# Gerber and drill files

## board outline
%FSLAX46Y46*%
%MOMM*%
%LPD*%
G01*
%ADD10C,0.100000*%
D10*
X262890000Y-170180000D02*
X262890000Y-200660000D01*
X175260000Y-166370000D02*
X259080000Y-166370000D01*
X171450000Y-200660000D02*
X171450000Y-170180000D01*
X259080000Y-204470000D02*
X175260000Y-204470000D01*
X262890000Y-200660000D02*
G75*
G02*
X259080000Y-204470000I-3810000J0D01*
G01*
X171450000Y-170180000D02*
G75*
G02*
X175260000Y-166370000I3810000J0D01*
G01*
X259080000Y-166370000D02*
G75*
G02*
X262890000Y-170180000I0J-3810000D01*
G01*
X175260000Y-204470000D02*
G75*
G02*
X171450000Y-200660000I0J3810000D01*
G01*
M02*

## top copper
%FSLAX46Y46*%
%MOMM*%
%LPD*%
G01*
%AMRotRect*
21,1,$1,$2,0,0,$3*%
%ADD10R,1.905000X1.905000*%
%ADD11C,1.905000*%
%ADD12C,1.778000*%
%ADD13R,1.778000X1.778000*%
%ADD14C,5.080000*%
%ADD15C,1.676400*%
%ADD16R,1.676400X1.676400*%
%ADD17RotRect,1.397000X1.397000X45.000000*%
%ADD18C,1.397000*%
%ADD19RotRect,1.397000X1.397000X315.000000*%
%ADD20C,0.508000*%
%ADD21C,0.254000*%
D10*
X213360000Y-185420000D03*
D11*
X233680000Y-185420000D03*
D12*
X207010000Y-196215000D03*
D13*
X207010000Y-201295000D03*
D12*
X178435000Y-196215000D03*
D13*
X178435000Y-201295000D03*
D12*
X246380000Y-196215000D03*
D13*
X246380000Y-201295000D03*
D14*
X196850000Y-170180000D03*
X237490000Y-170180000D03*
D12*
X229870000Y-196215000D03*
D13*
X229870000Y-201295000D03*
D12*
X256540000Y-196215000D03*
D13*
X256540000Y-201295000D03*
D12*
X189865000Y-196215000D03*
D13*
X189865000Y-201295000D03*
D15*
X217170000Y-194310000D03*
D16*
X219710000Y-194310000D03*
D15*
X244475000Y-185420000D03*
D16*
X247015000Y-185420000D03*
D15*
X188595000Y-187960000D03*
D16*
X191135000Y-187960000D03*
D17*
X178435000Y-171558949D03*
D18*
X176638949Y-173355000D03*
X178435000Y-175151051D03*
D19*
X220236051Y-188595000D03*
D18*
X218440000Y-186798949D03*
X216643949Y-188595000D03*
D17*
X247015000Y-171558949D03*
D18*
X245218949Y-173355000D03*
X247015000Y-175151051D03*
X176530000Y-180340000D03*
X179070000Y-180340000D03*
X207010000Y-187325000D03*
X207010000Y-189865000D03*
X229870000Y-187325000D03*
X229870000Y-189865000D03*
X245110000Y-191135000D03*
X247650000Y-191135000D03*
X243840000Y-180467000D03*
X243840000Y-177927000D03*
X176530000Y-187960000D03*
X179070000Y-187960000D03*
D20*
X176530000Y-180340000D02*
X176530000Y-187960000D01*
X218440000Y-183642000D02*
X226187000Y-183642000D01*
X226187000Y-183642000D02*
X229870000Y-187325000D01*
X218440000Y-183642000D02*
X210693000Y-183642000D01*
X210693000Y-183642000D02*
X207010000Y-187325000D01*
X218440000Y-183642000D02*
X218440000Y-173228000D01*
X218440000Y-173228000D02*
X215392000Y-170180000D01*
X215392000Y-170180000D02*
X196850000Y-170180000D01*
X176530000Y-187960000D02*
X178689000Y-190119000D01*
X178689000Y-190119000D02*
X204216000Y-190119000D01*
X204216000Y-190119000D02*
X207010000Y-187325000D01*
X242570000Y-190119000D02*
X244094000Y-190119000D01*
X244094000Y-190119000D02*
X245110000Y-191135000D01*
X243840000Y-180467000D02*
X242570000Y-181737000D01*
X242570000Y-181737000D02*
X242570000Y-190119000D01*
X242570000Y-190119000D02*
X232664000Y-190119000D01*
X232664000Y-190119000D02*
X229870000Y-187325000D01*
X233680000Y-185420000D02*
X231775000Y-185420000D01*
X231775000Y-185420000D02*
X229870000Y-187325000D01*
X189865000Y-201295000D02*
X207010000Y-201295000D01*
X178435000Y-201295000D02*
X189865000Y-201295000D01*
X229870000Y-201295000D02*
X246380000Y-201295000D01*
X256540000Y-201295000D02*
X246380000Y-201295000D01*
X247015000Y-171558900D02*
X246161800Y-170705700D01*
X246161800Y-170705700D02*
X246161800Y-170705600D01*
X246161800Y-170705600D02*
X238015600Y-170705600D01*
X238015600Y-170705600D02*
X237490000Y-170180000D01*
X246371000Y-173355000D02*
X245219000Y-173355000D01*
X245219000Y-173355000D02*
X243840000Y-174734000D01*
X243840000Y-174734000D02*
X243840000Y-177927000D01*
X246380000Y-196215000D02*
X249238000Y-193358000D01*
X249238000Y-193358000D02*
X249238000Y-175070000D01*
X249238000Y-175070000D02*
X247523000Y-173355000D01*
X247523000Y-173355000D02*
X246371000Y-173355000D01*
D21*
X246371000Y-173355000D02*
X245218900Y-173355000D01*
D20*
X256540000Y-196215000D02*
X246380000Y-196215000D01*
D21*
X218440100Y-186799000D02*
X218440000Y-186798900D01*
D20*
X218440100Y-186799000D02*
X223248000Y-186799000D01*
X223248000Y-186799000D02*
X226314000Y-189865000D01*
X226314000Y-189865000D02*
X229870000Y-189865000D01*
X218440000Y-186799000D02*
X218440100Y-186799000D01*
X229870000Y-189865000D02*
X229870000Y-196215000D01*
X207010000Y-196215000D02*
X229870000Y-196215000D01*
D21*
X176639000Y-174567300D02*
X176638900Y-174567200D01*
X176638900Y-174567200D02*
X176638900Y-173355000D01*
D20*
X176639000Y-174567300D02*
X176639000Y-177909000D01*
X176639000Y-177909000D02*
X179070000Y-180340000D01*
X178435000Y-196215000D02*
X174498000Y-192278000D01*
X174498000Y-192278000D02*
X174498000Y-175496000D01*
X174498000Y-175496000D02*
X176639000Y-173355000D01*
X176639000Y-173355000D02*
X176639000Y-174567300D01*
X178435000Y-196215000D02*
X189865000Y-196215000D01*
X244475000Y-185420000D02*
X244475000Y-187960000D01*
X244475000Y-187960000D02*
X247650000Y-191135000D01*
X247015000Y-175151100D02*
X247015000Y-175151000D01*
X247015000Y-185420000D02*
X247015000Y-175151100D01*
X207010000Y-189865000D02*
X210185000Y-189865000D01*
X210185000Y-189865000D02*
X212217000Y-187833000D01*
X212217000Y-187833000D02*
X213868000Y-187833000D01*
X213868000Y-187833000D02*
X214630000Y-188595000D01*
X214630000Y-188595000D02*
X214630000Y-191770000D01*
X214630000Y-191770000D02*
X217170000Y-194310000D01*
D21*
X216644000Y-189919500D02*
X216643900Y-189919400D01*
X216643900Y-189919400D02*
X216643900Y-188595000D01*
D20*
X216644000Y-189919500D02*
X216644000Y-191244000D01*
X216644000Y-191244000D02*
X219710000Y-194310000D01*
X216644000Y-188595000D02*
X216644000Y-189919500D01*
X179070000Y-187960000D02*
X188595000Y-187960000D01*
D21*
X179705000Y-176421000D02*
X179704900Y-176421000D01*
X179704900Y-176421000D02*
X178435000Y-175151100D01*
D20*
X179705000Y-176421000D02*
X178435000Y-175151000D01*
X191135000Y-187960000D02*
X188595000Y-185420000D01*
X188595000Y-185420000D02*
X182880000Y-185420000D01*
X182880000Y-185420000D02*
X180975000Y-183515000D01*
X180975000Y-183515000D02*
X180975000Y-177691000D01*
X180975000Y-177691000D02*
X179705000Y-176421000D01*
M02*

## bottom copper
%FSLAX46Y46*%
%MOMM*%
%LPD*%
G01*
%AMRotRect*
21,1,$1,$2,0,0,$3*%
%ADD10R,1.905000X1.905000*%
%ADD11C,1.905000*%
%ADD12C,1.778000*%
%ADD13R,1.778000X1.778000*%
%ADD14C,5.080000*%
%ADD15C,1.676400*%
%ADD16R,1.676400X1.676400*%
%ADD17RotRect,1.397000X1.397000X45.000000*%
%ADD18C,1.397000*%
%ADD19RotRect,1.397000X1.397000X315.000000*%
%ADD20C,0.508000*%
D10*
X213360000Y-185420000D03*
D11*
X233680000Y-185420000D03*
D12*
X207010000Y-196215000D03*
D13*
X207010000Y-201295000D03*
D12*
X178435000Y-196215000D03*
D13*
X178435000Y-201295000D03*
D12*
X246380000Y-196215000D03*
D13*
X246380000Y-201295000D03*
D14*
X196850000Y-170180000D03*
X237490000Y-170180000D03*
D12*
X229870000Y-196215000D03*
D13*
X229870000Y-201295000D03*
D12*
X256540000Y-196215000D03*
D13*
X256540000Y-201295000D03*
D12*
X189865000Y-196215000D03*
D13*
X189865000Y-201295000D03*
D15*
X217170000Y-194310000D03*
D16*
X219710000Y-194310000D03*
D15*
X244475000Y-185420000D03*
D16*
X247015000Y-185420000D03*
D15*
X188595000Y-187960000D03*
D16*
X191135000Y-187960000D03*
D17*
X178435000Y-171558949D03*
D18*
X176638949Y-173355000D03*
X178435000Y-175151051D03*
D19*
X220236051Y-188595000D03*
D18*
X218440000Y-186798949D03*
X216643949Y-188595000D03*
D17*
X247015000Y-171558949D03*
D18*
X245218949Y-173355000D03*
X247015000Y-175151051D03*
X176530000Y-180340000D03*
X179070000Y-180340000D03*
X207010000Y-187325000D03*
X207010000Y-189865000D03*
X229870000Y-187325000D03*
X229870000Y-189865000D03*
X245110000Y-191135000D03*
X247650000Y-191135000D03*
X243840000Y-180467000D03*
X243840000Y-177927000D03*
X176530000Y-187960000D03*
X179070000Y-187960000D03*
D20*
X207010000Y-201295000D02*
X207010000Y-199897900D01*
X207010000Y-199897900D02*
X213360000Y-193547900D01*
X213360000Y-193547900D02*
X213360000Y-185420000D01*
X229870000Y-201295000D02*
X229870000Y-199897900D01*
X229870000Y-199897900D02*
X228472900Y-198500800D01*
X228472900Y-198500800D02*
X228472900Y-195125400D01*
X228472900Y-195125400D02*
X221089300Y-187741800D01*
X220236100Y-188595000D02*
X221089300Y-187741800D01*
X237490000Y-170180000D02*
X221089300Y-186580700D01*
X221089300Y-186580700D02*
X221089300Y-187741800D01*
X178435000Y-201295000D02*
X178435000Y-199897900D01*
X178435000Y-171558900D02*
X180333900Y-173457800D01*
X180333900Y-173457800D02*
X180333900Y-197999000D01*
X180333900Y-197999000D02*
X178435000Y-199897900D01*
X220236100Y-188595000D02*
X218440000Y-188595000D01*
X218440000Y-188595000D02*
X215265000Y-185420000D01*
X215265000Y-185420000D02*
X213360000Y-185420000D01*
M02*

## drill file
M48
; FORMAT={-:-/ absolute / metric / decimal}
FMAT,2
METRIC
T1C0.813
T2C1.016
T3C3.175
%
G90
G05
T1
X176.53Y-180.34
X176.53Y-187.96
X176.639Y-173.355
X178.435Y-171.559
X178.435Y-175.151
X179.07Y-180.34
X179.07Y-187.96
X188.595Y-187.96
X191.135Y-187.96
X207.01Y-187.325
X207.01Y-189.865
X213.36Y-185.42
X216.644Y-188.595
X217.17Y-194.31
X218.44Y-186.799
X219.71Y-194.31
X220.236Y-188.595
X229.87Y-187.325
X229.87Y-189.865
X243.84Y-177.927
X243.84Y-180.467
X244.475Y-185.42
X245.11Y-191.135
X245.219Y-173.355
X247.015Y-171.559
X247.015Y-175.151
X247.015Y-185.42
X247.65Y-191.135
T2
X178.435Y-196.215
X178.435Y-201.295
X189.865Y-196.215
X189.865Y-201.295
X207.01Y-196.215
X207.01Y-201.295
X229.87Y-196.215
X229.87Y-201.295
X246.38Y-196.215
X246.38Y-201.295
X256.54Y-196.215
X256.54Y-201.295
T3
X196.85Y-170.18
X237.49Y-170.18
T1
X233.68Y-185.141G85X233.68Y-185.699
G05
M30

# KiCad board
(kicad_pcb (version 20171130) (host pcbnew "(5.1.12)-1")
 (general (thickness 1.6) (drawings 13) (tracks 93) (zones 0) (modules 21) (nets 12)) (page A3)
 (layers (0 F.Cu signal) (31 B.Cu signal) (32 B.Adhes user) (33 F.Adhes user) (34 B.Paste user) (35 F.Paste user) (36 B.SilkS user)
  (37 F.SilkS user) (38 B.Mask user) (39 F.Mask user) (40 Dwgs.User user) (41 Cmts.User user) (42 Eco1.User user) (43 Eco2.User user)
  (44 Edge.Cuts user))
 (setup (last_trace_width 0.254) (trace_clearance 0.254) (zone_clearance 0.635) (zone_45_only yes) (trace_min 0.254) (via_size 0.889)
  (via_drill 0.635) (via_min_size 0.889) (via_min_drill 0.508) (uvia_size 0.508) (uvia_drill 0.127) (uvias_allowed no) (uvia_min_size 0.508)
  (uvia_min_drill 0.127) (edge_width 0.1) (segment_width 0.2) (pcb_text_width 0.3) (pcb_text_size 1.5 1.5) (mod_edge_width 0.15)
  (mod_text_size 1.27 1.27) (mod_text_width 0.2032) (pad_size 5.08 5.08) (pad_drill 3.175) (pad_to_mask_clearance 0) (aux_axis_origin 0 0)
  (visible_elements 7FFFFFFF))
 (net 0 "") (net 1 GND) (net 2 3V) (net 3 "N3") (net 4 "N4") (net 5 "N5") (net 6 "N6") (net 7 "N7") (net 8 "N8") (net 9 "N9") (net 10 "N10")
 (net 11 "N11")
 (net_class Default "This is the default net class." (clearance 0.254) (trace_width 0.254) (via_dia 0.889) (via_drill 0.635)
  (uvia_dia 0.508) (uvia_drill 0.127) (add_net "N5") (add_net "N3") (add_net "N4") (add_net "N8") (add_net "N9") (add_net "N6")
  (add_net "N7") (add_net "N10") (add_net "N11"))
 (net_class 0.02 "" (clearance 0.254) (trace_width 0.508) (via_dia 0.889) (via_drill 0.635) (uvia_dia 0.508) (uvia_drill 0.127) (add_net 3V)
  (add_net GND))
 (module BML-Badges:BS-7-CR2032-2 (layer B.Cu) (at 217.17 185.42)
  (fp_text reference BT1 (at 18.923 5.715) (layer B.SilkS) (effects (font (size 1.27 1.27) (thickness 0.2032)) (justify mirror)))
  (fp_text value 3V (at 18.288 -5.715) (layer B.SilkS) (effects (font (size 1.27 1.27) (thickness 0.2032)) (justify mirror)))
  (pad 2 thru_hole rect (at -3.81 0) (size 1.905 1.905) (drill 0.8128) (layers *.Cu *.Mask B.SilkS) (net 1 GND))
  (pad 1 thru_hole circle (at 16.51 0) (size 1.905 1.905) (drill oval 0.8128 1.3716) (layers *.Cu *.Mask B.SilkS) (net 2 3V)))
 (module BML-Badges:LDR (layer F.Cu) (at 207.01 198.755 270)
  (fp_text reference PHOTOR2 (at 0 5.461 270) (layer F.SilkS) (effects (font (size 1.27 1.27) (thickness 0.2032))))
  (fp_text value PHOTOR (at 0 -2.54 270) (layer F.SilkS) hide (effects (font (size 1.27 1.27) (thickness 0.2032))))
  (pad 1 thru_hole circle (at -2.54 0 270) (size 1.778 1.778) (drill 1.016) (layers *.Cu *.Mask F.SilkS) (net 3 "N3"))
  (pad 2 thru_hole rect (at 2.54 0 270) (size 1.778 1.778) (drill 1.016) (layers *.Cu *.Mask F.SilkS) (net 1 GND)))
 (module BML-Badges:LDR (layer F.Cu) (at 178.435 198.755 270)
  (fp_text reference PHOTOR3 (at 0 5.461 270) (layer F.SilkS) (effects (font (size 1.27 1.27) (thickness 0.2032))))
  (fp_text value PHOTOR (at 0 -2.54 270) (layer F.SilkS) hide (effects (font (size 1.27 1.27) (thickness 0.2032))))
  (pad 1 thru_hole circle (at -2.54 0 270) (size 1.778 1.778) (drill 1.016) (layers *.Cu *.Mask F.SilkS) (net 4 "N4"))
  (pad 2 thru_hole rect (at 2.54 0 270) (size 1.778 1.778) (drill 1.016) (layers *.Cu *.Mask F.SilkS) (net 1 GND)))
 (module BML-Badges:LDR (layer F.Cu) (at 246.38 198.755 270)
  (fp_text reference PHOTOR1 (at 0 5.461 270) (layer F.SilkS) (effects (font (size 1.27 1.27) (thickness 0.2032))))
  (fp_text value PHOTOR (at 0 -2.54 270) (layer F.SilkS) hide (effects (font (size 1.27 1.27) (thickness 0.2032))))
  (pad 1 thru_hole circle (at -2.54 0 270) (size 1.778 1.778) (drill 1.016) (layers *.Cu *.Mask F.SilkS) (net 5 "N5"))
  (pad 2 thru_hole rect (at 2.54 0 270) (size 1.778 1.778) (drill 1.016) (layers *.Cu *.Mask F.SilkS) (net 1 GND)))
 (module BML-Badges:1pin (layer F.Cu) (at 196.85 170.18)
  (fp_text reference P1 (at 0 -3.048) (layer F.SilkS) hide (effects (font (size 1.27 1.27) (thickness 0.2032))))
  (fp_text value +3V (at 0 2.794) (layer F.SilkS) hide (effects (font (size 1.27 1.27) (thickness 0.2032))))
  (pad 1 thru_hole circle (at 0 0) (size 5.08 5.08) (drill 3.175) (layers *.Cu *.Mask F.SilkS) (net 2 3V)))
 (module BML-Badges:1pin (layer F.Cu) (at 237.49 170.18)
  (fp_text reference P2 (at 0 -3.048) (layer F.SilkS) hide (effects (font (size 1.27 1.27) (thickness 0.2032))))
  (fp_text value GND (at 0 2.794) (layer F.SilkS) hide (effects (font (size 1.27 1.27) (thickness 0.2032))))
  (pad 1 thru_hole circle (at 0 0) (size 5.08 5.08) (drill 3.175) (layers *.Cu *.Mask F.SilkS) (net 1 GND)))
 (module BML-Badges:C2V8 (layer F.Cu) (at 229.87 198.755 270)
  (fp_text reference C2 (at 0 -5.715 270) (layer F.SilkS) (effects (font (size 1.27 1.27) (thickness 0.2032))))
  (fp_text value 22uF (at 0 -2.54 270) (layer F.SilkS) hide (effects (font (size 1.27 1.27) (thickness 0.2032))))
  (pad 1 thru_hole circle (at -2.54 0 270) (size 1.778 1.778) (drill 1.016) (layers *.Cu *.Mask F.SilkS) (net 3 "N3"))
  (pad 2 thru_hole rect (at 2.54 0 270) (size 1.778 1.778) (drill 1.016) (layers *.Cu *.Mask F.SilkS) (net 1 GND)))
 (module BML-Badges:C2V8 (layer F.Cu) (at 256.54 198.755 270)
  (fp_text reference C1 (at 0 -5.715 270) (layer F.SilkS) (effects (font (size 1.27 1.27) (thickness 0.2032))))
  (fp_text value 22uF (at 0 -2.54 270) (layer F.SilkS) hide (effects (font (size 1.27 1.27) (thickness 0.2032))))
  (pad 1 thru_hole circle (at -2.54 0 270) (size 1.778 1.778) (drill 1.016) (layers *.Cu *.Mask F.SilkS) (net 5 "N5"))
  (pad 2 thru_hole rect (at 2.54 0 270) (size 1.778 1.778) (drill 1.016) (layers *.Cu *.Mask F.SilkS) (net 1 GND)))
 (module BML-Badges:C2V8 (layer F.Cu) (at 189.865 198.755 270)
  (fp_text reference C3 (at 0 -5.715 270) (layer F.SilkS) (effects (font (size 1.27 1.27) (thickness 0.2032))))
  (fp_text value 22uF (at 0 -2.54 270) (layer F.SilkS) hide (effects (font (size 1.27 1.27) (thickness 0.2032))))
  (pad 1 thru_hole circle (at -2.54 0 270) (size 1.778 1.778) (drill 1.016) (layers *.Cu *.Mask F.SilkS) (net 4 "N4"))
  (pad 2 thru_hole rect (at 2.54 0 270) (size 1.778 1.778) (drill 1.016) (layers *.Cu *.Mask F.SilkS) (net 1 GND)))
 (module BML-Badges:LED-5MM (layer F.Cu) (at 218.44 194.31)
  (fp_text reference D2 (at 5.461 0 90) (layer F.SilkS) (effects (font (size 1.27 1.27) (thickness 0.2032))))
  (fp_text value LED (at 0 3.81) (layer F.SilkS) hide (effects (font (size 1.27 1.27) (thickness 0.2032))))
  (pad 1 thru_hole circle (at -1.27 0) (size 1.6764 1.6764) (drill 0.8128) (layers *.Cu *.Mask F.SilkS) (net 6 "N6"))
  (pad 2 thru_hole rect (at 1.27 0) (size 1.6764 1.6764) (drill 0.8128) (layers *.Cu *.Mask F.SilkS) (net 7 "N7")))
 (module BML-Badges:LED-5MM (layer F.Cu) (at 245.745 185.42)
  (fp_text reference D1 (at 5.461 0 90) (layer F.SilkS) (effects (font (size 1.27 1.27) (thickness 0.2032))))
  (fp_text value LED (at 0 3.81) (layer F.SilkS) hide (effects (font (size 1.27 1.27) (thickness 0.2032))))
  (pad 1 thru_hole circle (at -1.27 0) (size 1.6764 1.6764) (drill 0.8128) (layers *.Cu *.Mask F.SilkS) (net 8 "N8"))
  (pad 2 thru_hole rect (at 1.27 0) (size 1.6764 1.6764) (drill 0.8128) (layers *.Cu *.Mask F.SilkS) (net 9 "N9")))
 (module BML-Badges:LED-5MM (layer F.Cu) (at 189.865 187.96)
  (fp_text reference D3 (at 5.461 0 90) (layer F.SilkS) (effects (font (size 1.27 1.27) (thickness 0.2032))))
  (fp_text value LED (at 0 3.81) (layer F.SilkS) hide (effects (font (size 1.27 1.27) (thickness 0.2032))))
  (pad 1 thru_hole circle (at -1.27 0) (size 1.6764 1.6764) (drill 0.8128) (layers *.Cu *.Mask F.SilkS) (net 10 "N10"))
  (pad 2 thru_hole rect (at 1.27 0) (size 1.6764 1.6764) (drill 0.8128) (layers *.Cu *.Mask F.SilkS) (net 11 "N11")))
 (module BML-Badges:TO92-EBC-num (layer F.Cu) (at 178.435 173.355 45)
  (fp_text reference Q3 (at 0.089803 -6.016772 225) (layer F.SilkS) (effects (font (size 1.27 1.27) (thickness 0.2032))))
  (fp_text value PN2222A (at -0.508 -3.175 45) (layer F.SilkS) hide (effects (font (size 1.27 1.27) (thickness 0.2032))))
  (pad 1 thru_hole rect (at 1.27 -1.27 45) (size 1.397 1.397) (drill 0.8128) (layers *.Cu *.Mask F.SilkS) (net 1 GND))
  (pad 2 thru_hole circle (at -1.27 -1.27 45) (size 1.397 1.397) (drill 0.8128) (layers *.Cu *.Mask F.SilkS) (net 4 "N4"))
  (pad 3 thru_hole circle (at -1.27 1.27 45) (size 1.397 1.397) (drill 0.8128) (layers *.Cu *.Mask F.SilkS) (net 11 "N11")))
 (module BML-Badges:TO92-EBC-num (layer F.Cu) (at 218.44 188.595 315)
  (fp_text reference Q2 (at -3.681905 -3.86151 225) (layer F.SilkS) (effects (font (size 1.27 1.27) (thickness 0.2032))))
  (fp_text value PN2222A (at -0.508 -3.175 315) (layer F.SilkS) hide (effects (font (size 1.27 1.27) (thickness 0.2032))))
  (pad 1 thru_hole rect (at 1.27 -1.27 315) (size 1.397 1.397) (drill 0.8128) (layers *.Cu *.Mask F.SilkS) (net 1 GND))
  (pad 2 thru_hole circle (at -1.27 -1.27 315) (size 1.397 1.397) (drill 0.8128) (layers *.Cu *.Mask F.SilkS) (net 3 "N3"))
  (pad 3 thru_hole circle (at -1.27 1.27 315) (size 1.397 1.397) (drill 0.8128) (layers *.Cu *.Mask F.SilkS) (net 7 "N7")))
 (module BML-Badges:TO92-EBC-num (layer F.Cu) (at 247.015 173.355 45)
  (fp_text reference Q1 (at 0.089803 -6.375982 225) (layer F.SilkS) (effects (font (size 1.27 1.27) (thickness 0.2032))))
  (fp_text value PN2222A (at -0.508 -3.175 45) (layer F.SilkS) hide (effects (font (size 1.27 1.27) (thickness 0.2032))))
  (pad 1 thru_hole rect (at 1.27 -1.27 45) (size 1.397 1.397) (drill 0.8128) (layers *.Cu *.Mask F.SilkS) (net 1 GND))
  (pad 2 thru_hole circle (at -1.27 -1.27 45) (size 1.397 1.397) (drill 0.8128) (layers *.Cu *.Mask F.SilkS) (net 5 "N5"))
  (pad 3 thru_hole circle (at -1.27 1.27 45) (size 1.397 1.397) (drill 0.8128) (layers *.Cu *.Mask F.SilkS) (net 9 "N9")))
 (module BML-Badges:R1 (layer F.Cu) (at 177.8 180.34) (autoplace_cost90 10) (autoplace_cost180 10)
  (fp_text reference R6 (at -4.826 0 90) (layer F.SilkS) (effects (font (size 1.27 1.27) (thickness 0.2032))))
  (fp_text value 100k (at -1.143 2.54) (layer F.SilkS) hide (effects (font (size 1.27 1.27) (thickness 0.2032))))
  (pad 1 thru_hole circle (at -1.27 0) (size 1.397 1.397) (drill 0.8128) (layers *.Cu *.Mask F.SilkS) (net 2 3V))
  (pad 2 thru_hole circle (at 1.27 0) (size 1.397 1.397) (drill 0.8128) (layers *.Cu *.Mask F.SilkS) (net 4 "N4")))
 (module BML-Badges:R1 (layer F.Cu) (at 207.01 188.595 270) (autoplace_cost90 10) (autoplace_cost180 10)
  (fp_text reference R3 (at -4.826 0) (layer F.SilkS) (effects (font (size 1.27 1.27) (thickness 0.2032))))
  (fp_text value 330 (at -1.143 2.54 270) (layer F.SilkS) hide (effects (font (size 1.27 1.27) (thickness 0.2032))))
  (pad 1 thru_hole circle (at -1.27 0 270) (size 1.397 1.397) (drill 0.8128) (layers *.Cu *.Mask F.SilkS) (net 2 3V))
  (pad 2 thru_hole circle (at 1.27 0 270) (size 1.397 1.397) (drill 0.8128) (layers *.Cu *.Mask F.SilkS) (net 6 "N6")))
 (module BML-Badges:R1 (layer F.Cu) (at 229.87 188.595 270) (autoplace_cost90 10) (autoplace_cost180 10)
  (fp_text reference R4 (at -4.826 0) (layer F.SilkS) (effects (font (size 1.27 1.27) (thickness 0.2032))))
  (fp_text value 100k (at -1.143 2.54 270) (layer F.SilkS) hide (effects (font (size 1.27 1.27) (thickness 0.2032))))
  (pad 1 thru_hole circle (at -1.27 0 270) (size 1.397 1.397) (drill 0.8128) (layers *.Cu *.Mask F.SilkS) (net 2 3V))
  (pad 2 thru_hole circle (at 1.27 0 270) (size 1.397 1.397) (drill 0.8128) (layers *.Cu *.Mask F.SilkS) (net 3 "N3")))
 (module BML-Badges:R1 (layer F.Cu) (at 246.38 191.135) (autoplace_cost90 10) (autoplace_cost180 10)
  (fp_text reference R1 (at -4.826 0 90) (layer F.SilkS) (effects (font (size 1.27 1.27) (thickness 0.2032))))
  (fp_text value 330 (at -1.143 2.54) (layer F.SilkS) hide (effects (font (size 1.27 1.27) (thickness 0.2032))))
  (pad 1 thru_hole circle (at -1.27 0) (size 1.397 1.397) (drill 0.8128) (layers *.Cu *.Mask F.SilkS) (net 2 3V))
  (pad 2 thru_hole circle (at 1.27 0) (size 1.397 1.397) (drill 0.8128) (layers *.Cu *.Mask F.SilkS) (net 8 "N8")))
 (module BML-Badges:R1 (layer F.Cu) (at 243.84 179.197 90) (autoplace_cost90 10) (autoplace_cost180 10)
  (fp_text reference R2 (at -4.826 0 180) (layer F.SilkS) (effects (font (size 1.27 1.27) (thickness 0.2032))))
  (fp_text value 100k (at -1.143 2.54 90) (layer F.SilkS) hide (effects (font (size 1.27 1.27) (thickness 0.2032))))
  (pad 1 thru_hole circle (at -1.27 0 90) (size 1.397 1.397) (drill 0.8128) (layers *.Cu *.Mask F.SilkS) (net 2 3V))
  (pad 2 thru_hole circle (at 1.27 0 90) (size 1.397 1.397) (drill 0.8128) (layers *.Cu *.Mask F.SilkS) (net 5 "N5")))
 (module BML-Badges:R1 (layer F.Cu) (at 177.8 187.96) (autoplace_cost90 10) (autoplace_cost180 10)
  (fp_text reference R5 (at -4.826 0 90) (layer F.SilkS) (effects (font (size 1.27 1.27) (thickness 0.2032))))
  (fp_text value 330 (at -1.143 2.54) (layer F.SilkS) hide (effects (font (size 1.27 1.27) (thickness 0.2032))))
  (pad 1 thru_hole circle (at -1.27 0) (size 1.397 1.397) (drill 0.8128) (layers *.Cu *.Mask F.SilkS) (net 2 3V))
  (pad 2 thru_hole circle (at 1.27 0) (size 1.397 1.397) (drill 0.8128) (layers *.Cu *.Mask F.SilkS) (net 10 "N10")))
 (gr_line (start 262.89 170.18) (end 262.89 200.66) (angle 90) (layer Edge.Cuts) (width 0.1))
 (gr_line (start 175.26 166.37) (end 259.08 166.37) (angle 90) (layer Edge.Cuts) (width 0.1))
 (gr_line (start 171.45 200.66) (end 171.45 170.18) (angle 90) (layer Edge.Cuts) (width 0.1))
 (gr_line (start 259.08 204.47) (end 175.26 204.47) (angle 90) (layer Edge.Cuts) (width 0.1))
 (gr_arc (start 259.08 200.66) (end 262.89 200.66) (angle 90) (layer Edge.Cuts) (width 0.1))
 (gr_arc (start 175.26 170.18) (end 171.45 170.18) (angle 90) (layer Edge.Cuts) (width 0.1))
 (gr_arc (start 259.08 170.18) (end 259.08 166.37) (angle 90) (layer Edge.Cuts) (width 0.1))
 (gr_arc (start 175.26 200.66) (end 175.26 204.47) (angle 90) (layer Edge.Cuts) (width 0.1))
 (segment (start 176.53 180.34) (end 176.53 187.96) (width 0.508) (layer F.Cu) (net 2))
 (segment (start 218.44 183.642) (end 226.187 183.642) (width 0.508) (layer F.Cu) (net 2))
 (segment (start 226.187 183.642) (end 229.87 187.325) (width 0.508) (layer F.Cu) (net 2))
 (segment (start 218.44 183.642) (end 210.693 183.642) (width 0.508) (layer F.Cu) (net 2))
 (segment (start 210.693 183.642) (end 207.01 187.325) (width 0.508) (layer F.Cu) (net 2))
 (segment (start 218.44 183.642) (end 218.44 173.228) (width 0.508) (layer F.Cu) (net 2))
 (segment (start 218.44 173.228) (end 215.392 170.18) (width 0.508) (layer F.Cu) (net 2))
 (segment (start 215.392 170.18) (end 196.85 170.18) (width 0.508) (layer F.Cu) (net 2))
 (segment (start 176.53 187.96) (end 178.689 190.119) (width 0.508) (layer F.Cu) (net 2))
 (segment (start 178.689 190.119) (end 204.216 190.119) (width 0.508) (layer F.Cu) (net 2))
 (segment (start 204.216 190.119) (end 207.01 187.325) (width 0.508) (layer F.Cu) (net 2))
 (segment (start 242.57 190.119) (end 244.094 190.119) (width 0.508) (layer F.Cu) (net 2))
 (segment (start 244.094 190.119) (end 245.11 191.135) (width 0.508) (layer F.Cu) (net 2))
 (segment (start 243.84 180.467) (end 242.57 181.737) (width 0.508) (layer F.Cu) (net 2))
 (segment (start 242.57 181.737) (end 242.57 190.119) (width 0.508) (layer F.Cu) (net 2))
 (segment (start 242.57 190.119) (end 232.664 190.119) (width 0.508) (layer F.Cu) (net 2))
 (segment (start 232.664 190.119) (end 229.87 187.325) (width 0.508) (layer F.Cu) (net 2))
 (segment (start 233.68 185.42) (end 231.775 185.42) (width 0.508) (layer F.Cu) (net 2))
 (segment (start 231.775 185.42) (end 229.87 187.325) (width 0.508) (layer F.Cu) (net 2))
 (segment (start 207.01 201.295) (end 207.01 199.8979) (width 0.508) (layer B.Cu) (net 1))
 (segment (start 207.01 199.8979) (end 213.36 193.5479) (width 0.508) (layer B.Cu) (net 1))
 (segment (start 213.36 193.5479) (end 213.36 185.42) (width 0.508) (layer B.Cu) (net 1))
 (segment (start 189.865 201.295) (end 207.01 201.295) (width 0.508) (layer F.Cu) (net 1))
 (segment (start 178.435 201.295) (end 189.865 201.295) (width 0.508) (layer F.Cu) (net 1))
 (segment (start 229.87 201.295) (end 229.87 199.8979) (width 0.508) (layer B.Cu) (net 1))
 (segment (start 229.87 199.8979) (end 228.4729 198.5008) (width 0.508) (layer B.Cu) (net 1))
 (segment (start 228.4729 198.5008) (end 228.4729 195.1254) (width 0.508) (layer B.Cu) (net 1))
 (segment (start 228.4729 195.1254) (end 221.0893 187.7418) (width 0.508) (layer B.Cu) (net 1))
 (segment (start 229.87 201.295) (end 246.38 201.295) (width 0.508) (layer F.Cu) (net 1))
 (segment (start 256.54 201.295) (end 246.38 201.295) (width 0.508) (layer F.Cu) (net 1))
 (segment (start 220.2361 188.595) (end 221.0893 187.7418) (width 0.508) (layer B.Cu) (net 1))
 (segment (start 237.49 170.18) (end 221.0893 186.5807) (width 0.508) (layer B.Cu) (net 1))
 (segment (start 221.0893 186.5807) (end 221.0893 187.7418) (width 0.508) (layer B.Cu) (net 1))
 (segment (start 178.435 201.295) (end 178.435 199.8979) (width 0.508) (layer B.Cu) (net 1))
 (segment (start 178.435 171.5589) (end 180.3339 173.4578) (width 0.508) (layer B.Cu) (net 1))
 (segment (start 180.3339 173.4578) (end 180.3339 197.999) (width 0.508) (layer B.Cu) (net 1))
 (segment (start 180.3339 197.999) (end 178.435 199.8979) (width 0.508) (layer B.Cu) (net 1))
 (segment (start 220.2361 188.595) (end 218.44 188.595) (width 0.508) (layer B.Cu) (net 1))
 (segment (start 218.44 188.595) (end 215.265 185.42) (width 0.508) (layer B.Cu) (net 1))
 (segment (start 215.265 185.42) (end 213.36 185.42) (width 0.508) (layer B.Cu) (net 1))
 (segment (start 247.015 171.5589) (end 246.1618 170.7057) (width 0.508) (layer F.Cu) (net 1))
 (segment (start 246.1618 170.7057) (end 246.1618 170.7056) (width 0.508) (layer F.Cu) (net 1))
 (segment (start 246.1618 170.7056) (end 238.0156 170.7056) (width 0.508) (layer F.Cu) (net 1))
 (segment (start 238.0156 170.7056) (end 237.49 170.18) (width 0.508) (layer F.Cu) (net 1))
 (segment (start 246.371 173.355) (end 245.219 173.355) (width 0.508) (layer F.Cu) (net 5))
 (segment (start 245.219 173.355) (end 243.84 174.734) (width 0.508) (layer F.Cu) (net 5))
 (segment (start 243.84 174.734) (end 243.84 177.927) (width 0.508) (layer F.Cu) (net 5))
 (segment (start 246.38 196.215) (end 249.238 193.358) (width 0.508) (layer F.Cu) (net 5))
 (segment (start 249.238 193.358) (end 249.238 175.07) (width 0.508) (layer F.Cu) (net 5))
 (segment (start 249.238 175.07) (end 247.523 173.355) (width 0.508) (layer F.Cu) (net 5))
 (segment (start 247.523 173.355) (end 246.371 173.355) (width 0.508) (layer F.Cu) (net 5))
 (segment (start 246.371 173.355) (end 245.2189 173.355) (width 0.254) (layer F.Cu) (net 5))
 (segment (start 256.54 196.215) (end 246.38 196.215) (width 0.508) (layer F.Cu) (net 5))
 (segment (start 218.4401 186.799) (end 218.44 186.7989) (width 0.254) (layer F.Cu) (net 3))
 (segment (start 218.4401 186.799) (end 223.248 186.799) (width 0.508) (layer F.Cu) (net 3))
 (segment (start 223.248 186.799) (end 226.314 189.865) (width 0.508) (layer F.Cu) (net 3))
 (segment (start 226.314 189.865) (end 229.87 189.865) (width 0.508) (layer F.Cu) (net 3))
 (segment (start 218.44 186.799) (end 218.4401 186.799) (width 0.508) (layer F.Cu) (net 3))
 (segment (start 229.87 189.865) (end 229.87 196.215) (width 0.508) (layer F.Cu) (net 3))
 (segment (start 207.01 196.215) (end 229.87 196.215) (width 0.508) (layer F.Cu) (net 3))
 (segment (start 176.639 174.5673) (end 176.6389 174.5672) (width 0.254) (layer F.Cu) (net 4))
 (segment (start 176.6389 174.5672) (end 176.6389 173.355) (width 0.254) (layer F.Cu) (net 4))
 (segment (start 176.639 174.5673) (end 176.639 177.909) (width 0.508) (layer F.Cu) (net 4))
 (segment (start 176.639 177.909) (end 179.07 180.34) (width 0.508) (layer F.Cu) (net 4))
 (segment (start 178.435 196.215) (end 174.498 192.278) (width 0.508) (layer F.Cu) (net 4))
 (segment (start 174.498 192.278) (end 174.498 175.496) (width 0.508) (layer F.Cu) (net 4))
 (segment (start 174.498 175.496) (end 176.639 173.355) (width 0.508) (layer F.Cu) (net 4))
 (segment (start 176.639 173.355) (end 176.639 174.5673) (width 0.508) (layer F.Cu) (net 4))
 (segment (start 178.435 196.215) (end 189.865 196.215) (width 0.508) (layer F.Cu) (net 4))
 (segment (start 244.475 185.42) (end 244.475 187.96) (width 0.508) (layer F.Cu) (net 8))
 (segment (start 244.475 187.96) (end 247.65 191.135) (width 0.508) (layer F.Cu) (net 8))
 (segment (start 247.015 175.1511) (end 247.015 175.151) (width 0.508) (layer F.Cu) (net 9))
 (segment (start 247.015 185.42) (end 247.015 175.1511) (width 0.508) (layer F.Cu) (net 9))
 (segment (start 207.01 189.865) (end 210.185 189.865) (width 0.508) (layer F.Cu) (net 6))
 (segment (start 210.185 189.865) (end 212.217 187.833) (width 0.508) (layer F.Cu) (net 6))
 (segment (start 212.217 187.833) (end 213.868 187.833) (width 0.508) (layer F.Cu) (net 6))
 (segment (start 213.868 187.833) (end 214.63 188.595) (width 0.508) (layer F.Cu) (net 6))
 (segment (start 214.63 188.595) (end 214.63 191.77) (width 0.508) (layer F.Cu) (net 6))
 (segment (start 214.63 191.77) (end 217.17 194.31) (width 0.508) (layer F.Cu) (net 6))
 (segment (start 216.644 189.9195) (end 216.6439 189.9194) (width 0.254) (layer F.Cu) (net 7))
 (segment (start 216.6439 189.9194) (end 216.6439 188.595) (width 0.254) (layer F.Cu) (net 7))
 (segment (start 216.644 189.9195) (end 216.644 191.244) (width 0.508) (layer F.Cu) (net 7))
 (segment (start 216.644 191.244) (end 219.71 194.31) (width 0.508) (layer F.Cu) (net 7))
 (segment (start 216.644 188.595) (end 216.644 189.9195) (width 0.508) (layer F.Cu) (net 7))
 (segment (start 179.07 187.96) (end 188.595 187.96) (width 0.508) (layer F.Cu) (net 10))
 (segment (start 179.705 176.421) (end 179.7049 176.421) (width 0.254) (layer F.Cu) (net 11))
 (segment (start 179.7049 176.421) (end 178.435 175.1511) (width 0.254) (layer F.Cu) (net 11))
 (segment (start 179.705 176.421) (end 178.435 175.151) (width 0.508) (layer F.Cu) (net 11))
 (segment (start 191.135 187.96) (end 188.595 185.42) (width 0.508) (layer F.Cu) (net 11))
 (segment (start 188.595 185.42) (end 182.88 185.42) (width 0.508) (layer F.Cu) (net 11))
 (segment (start 182.88 185.42) (end 180.975 183.515) (width 0.508) (layer F.Cu) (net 11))
 (segment (start 180.975 183.515) (end 180.975 177.691) (width 0.508) (layer F.Cu) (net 11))
 (segment (start 180.975 177.691) (end 179.705 176.421) (width 0.508) (layer F.Cu) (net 11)))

